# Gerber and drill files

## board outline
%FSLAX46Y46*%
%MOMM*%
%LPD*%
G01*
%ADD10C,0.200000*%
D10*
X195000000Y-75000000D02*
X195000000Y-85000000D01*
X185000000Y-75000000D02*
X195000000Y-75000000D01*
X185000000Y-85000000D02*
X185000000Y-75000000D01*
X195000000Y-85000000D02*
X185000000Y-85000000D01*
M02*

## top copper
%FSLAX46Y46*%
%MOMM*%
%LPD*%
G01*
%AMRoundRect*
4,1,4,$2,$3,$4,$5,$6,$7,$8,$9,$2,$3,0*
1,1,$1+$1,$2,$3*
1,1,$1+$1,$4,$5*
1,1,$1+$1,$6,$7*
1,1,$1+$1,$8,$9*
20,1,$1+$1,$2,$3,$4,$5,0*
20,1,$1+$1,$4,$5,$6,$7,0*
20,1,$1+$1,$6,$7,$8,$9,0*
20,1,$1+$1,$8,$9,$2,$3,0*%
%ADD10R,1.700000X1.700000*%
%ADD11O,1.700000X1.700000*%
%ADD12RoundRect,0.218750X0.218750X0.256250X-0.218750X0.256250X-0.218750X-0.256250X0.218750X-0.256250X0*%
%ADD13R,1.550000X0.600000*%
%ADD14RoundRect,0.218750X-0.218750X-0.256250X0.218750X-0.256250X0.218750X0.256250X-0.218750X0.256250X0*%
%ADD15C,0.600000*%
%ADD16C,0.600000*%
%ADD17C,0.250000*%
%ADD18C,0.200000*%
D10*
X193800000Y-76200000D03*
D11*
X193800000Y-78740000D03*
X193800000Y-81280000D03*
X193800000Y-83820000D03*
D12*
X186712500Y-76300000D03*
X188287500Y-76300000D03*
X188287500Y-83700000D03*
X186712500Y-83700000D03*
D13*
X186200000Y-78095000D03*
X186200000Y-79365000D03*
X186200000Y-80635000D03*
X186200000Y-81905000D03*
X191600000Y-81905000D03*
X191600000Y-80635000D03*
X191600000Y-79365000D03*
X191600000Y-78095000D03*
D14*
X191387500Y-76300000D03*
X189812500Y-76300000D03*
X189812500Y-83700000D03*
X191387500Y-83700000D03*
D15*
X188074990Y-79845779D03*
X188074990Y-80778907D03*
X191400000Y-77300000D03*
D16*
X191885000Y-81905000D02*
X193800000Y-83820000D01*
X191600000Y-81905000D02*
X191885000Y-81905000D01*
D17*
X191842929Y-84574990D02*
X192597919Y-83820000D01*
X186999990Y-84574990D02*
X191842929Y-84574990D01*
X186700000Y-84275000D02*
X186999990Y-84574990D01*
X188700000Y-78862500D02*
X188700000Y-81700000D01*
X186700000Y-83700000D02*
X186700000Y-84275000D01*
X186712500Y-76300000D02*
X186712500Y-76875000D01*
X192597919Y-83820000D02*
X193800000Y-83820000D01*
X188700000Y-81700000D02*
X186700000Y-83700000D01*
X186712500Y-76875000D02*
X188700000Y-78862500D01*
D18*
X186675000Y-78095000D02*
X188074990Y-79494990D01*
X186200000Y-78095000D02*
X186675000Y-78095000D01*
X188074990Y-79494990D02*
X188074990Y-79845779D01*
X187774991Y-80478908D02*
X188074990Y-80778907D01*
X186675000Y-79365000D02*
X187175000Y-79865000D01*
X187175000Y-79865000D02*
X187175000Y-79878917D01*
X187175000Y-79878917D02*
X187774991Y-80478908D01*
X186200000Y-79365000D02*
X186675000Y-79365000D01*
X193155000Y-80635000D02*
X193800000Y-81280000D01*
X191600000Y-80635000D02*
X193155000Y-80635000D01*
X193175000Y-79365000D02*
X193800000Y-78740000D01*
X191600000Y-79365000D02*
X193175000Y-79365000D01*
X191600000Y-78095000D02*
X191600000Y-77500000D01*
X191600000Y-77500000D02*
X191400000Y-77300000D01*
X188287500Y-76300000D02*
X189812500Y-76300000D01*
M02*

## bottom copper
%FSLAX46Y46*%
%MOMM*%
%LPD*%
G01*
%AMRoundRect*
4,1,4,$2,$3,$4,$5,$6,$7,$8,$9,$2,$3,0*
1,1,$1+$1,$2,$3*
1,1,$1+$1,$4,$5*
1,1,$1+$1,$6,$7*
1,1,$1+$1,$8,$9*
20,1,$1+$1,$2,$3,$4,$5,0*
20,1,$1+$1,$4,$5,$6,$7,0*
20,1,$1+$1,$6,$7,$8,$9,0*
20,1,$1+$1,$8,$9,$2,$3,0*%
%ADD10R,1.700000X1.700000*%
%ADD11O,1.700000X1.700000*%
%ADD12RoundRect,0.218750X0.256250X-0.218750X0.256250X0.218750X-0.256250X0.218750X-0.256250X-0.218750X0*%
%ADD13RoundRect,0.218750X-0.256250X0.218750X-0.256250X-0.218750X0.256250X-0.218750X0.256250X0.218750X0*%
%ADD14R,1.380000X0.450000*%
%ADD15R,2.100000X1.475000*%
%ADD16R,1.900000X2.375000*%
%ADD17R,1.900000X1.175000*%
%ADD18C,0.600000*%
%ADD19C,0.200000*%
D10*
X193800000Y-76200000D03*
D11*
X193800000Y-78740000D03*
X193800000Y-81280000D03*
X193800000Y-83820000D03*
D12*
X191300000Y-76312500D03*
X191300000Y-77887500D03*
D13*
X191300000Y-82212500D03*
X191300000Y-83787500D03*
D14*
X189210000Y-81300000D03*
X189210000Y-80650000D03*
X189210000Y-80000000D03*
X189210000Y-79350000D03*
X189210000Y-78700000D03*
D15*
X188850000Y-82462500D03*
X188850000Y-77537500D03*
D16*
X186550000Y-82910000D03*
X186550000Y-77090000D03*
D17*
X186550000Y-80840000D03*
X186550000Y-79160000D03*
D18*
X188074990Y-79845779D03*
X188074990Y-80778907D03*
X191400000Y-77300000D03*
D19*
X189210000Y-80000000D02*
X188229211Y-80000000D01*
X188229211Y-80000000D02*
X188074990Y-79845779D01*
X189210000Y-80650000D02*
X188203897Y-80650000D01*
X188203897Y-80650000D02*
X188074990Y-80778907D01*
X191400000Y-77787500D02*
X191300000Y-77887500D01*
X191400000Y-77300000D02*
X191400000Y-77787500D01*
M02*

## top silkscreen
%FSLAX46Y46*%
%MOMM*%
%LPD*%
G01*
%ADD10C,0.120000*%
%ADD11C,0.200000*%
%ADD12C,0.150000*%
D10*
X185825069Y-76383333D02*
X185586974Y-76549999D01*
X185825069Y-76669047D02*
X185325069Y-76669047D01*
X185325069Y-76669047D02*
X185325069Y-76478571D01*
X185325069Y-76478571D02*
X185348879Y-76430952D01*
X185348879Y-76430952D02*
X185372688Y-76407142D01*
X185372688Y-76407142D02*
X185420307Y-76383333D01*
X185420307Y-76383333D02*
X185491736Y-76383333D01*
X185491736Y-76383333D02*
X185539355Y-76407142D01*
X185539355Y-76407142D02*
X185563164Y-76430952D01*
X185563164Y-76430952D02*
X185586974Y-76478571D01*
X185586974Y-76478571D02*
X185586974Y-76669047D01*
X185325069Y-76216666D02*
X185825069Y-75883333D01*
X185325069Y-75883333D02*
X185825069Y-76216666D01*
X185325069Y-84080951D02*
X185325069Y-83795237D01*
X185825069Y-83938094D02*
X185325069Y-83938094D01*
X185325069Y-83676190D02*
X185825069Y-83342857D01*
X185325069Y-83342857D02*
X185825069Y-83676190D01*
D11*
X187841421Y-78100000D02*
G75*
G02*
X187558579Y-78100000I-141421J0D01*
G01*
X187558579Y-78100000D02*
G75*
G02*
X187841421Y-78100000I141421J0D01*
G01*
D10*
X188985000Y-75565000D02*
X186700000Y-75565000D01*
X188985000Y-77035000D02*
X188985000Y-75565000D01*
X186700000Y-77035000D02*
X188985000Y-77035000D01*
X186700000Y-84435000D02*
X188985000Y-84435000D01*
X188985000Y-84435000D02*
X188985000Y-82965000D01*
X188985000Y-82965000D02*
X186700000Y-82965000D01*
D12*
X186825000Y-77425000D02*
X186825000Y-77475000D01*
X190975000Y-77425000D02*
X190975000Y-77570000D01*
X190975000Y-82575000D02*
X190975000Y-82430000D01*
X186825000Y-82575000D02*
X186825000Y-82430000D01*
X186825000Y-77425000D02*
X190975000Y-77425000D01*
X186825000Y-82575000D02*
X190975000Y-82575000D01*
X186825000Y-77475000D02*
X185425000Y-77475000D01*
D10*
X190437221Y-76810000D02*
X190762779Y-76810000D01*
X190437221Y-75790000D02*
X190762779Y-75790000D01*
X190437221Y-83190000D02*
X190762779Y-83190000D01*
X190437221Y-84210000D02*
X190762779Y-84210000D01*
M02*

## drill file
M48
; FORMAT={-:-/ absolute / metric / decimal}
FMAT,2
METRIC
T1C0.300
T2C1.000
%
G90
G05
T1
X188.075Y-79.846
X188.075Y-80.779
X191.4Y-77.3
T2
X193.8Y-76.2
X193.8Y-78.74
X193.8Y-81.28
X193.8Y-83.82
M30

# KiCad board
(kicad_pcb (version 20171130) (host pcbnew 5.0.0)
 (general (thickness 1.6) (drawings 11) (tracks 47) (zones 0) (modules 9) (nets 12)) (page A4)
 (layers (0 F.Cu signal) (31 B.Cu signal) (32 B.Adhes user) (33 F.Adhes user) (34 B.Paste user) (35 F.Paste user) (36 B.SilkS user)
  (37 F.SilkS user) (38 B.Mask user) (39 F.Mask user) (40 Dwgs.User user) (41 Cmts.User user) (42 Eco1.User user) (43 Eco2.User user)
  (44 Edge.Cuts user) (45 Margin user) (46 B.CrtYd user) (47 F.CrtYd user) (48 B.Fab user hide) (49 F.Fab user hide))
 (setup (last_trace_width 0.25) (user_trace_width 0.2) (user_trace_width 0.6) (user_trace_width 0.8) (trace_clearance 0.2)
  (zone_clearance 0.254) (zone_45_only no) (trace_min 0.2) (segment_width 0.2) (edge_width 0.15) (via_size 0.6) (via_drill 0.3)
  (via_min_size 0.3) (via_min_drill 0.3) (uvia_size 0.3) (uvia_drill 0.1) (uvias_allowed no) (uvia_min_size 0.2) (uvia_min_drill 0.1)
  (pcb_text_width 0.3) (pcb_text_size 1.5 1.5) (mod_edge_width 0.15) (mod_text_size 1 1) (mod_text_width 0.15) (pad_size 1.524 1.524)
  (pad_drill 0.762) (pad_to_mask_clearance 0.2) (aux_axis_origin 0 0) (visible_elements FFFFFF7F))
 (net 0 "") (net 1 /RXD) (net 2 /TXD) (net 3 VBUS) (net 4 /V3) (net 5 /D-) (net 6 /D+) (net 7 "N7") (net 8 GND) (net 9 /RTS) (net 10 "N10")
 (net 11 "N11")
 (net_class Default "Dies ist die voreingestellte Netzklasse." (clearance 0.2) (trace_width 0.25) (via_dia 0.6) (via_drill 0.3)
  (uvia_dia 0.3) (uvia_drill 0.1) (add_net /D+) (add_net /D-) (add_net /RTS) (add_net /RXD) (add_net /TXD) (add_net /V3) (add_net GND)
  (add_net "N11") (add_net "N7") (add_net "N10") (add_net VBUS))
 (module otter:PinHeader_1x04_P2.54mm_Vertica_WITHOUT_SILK (layer F.Cu) (at 193.8 76.2)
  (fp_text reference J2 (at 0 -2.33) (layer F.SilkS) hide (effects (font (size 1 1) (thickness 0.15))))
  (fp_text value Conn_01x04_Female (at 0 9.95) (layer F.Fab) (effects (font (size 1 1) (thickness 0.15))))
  (pad 1 thru_hole rect (at 0 0) (size 1.7 1.7) (drill 1) (layers *.Cu *.Mask))
  (pad 2 thru_hole oval (at 0 2.54) (size 1.7 1.7) (drill 1) (layers *.Cu *.Mask) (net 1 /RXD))
  (pad 3 thru_hole oval (at 0 5.08) (size 1.7 1.7) (drill 1) (layers *.Cu *.Mask) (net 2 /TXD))
  (pad 4 thru_hole oval (at 0 7.62) (size 1.7 1.7) (drill 1) (layers *.Cu *.Mask) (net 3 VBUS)))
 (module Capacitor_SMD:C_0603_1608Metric (layer B.Cu) (at 191.3 77.1 90)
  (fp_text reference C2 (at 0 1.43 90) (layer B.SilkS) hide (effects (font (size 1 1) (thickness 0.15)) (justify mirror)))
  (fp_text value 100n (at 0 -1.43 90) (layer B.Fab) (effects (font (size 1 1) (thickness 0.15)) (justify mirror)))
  (pad 2 smd roundrect (at 0.7875 0 90) (size 0.875 0.95) (layers B.Cu B.Paste B.Mask) (roundrect_rratio 0.25))
  (pad 1 smd roundrect (at -0.7875 0 90) (size 0.875 0.95) (layers B.Cu B.Paste B.Mask) (roundrect_rratio 0.25) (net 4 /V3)))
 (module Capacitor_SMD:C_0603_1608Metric (layer B.Cu) (at 191.3 83 270)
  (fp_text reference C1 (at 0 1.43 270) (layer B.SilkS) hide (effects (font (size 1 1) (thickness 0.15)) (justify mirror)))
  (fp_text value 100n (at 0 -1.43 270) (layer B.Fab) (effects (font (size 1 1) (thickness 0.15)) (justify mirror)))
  (pad 1 smd roundrect (at -0.7875 0 270) (size 0.875 0.95) (layers B.Cu B.Paste B.Mask) (roundrect_rratio 0.25))
  (pad 2 smd roundrect (at 0.7875 0 270) (size 0.875 0.95) (layers B.Cu B.Paste B.Mask) (roundrect_rratio 0.25)))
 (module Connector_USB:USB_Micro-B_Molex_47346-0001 (layer B.Cu) (at 187.75 80 90)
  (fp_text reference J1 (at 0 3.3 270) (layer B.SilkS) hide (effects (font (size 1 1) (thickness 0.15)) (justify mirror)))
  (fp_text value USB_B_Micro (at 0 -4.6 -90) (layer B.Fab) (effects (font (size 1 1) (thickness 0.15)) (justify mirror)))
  (pad 1 smd rect (at -1.3 1.46 90) (size 0.45 1.38) (layers B.Cu B.Paste B.Mask))
  (pad 2 smd rect (at -0.65 1.46 90) (size 0.45 1.38) (layers B.Cu B.Paste B.Mask) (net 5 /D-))
  (pad 3 smd rect (at 0 1.46 90) (size 0.45 1.38) (layers B.Cu B.Paste B.Mask) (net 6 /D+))
  (pad 4 smd rect (at 0.65 1.46 90) (size 0.45 1.38) (layers B.Cu B.Paste B.Mask))
  (pad 5 smd rect (at 1.3 1.46 90) (size 0.45 1.38) (layers B.Cu B.Paste B.Mask))
  (pad 6 smd rect (at -2.4625 1.1 90) (size 1.475 2.1) (layers B.Cu B.Paste B.Mask))
  (pad 6 smd rect (at 2.4625 1.1 90) (size 1.475 2.1) (layers B.Cu B.Paste B.Mask))
  (pad 6 smd rect (at -2.91 -1.2 90) (size 2.375 1.9) (layers B.Cu B.Paste B.Mask))
  (pad 6 smd rect (at 2.91 -1.2 90) (size 2.375 1.9) (layers B.Cu B.Paste B.Mask))
  (pad 6 smd rect (at -0.84 -1.2 90) (size 1.175 1.9) (layers B.Cu B.Paste B.Mask))
  (pad 6 smd rect (at 0.84 -1.2 90) (size 1.175 1.9) (layers B.Cu B.Paste B.Mask)))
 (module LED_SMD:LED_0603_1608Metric (layer F.Cu) (at 187.5 76.3 180)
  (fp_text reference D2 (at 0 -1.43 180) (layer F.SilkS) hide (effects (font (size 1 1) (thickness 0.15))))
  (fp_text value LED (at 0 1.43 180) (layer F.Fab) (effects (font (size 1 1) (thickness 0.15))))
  (fp_line (start -1.485 0.735) (end 0.8 0.735) (layer F.SilkS) (width 0.12))
  (fp_line (start -1.485 -0.735) (end -1.485 0.735) (layer F.SilkS) (width 0.12))
  (fp_line (start 0.8 -0.735) (end -1.485 -0.735) (layer F.SilkS) (width 0.12))
  (pad 2 smd roundrect (at 0.7875 0 180) (size 0.875 0.95) (layers F.Cu F.Paste F.Mask) (roundrect_rratio 0.25) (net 3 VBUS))
  (pad 1 smd roundrect (at -0.7875 0 180) (size 0.875 0.95) (layers F.Cu F.Paste F.Mask) (roundrect_rratio 0.25) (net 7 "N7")))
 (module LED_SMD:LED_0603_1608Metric (layer F.Cu) (at 187.5 83.7 180)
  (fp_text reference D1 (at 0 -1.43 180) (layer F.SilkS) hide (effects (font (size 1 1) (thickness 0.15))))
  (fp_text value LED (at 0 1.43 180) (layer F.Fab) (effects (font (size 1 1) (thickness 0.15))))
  (fp_line (start 0.8 -0.735) (end -1.485 -0.735) (layer F.SilkS) (width 0.12))
  (fp_line (start -1.485 -0.735) (end -1.485 0.735) (layer F.SilkS) (width 0.12))
  (fp_line (start -1.485 0.735) (end 0.8 0.735) (layer F.SilkS) (width 0.12))
  (pad 1 smd roundrect (at -0.7875 0 180) (size 0.875 0.95) (layers F.Cu F.Paste F.Mask) (roundrect_rratio 0.25))
  (pad 2 smd roundrect (at 0.7875 0 180) (size 0.875 0.95) (layers F.Cu F.Paste F.Mask) (roundrect_rratio 0.25)))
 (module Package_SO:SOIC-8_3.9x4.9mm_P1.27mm (layer F.Cu) (at 188.9 80)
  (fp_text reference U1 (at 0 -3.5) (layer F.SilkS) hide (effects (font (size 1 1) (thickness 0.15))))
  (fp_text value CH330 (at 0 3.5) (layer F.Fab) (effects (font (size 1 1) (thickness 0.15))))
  (fp_line (start -2.075 -2.575) (end -2.075 -2.525) (layer F.SilkS) (width 0.15))
  (fp_line (start 2.075 -2.575) (end 2.075 -2.43) (layer F.SilkS) (width 0.15))
  (fp_line (start 2.075 2.575) (end 2.075 2.43) (layer F.SilkS) (width 0.15))
  (fp_line (start -2.075 2.575) (end -2.075 2.43) (layer F.SilkS) (width 0.15))
  (fp_line (start -2.075 -2.575) (end 2.075 -2.575) (layer F.SilkS) (width 0.15))
  (fp_line (start -2.075 2.575) (end 2.075 2.575) (layer F.SilkS) (width 0.15))
  (fp_line (start -2.075 -2.525) (end -3.475 -2.525) (layer F.SilkS) (width 0.15))
  (pad 1 smd rect (at -2.7 -1.905) (size 1.55 0.6) (layers F.Cu F.Paste F.Mask) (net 6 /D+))
  (pad 2 smd rect (at -2.7 -0.635) (size 1.55 0.6) (layers F.Cu F.Paste F.Mask) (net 5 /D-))
  (pad 3 smd rect (at -2.7 0.635) (size 1.55 0.6) (layers F.Cu F.Paste F.Mask))
  (pad 4 smd rect (at -2.7 1.905) (size 1.55 0.6) (layers F.Cu F.Paste F.Mask))
  (pad 5 smd rect (at 2.7 1.905) (size 1.55 0.6) (layers F.Cu F.Paste F.Mask) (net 3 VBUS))
  (pad 6 smd rect (at 2.7 0.635) (size 1.55 0.6) (layers F.Cu F.Paste F.Mask) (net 2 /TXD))
  (pad 7 smd rect (at 2.7 -0.635) (size 1.55 0.6) (layers F.Cu F.Paste F.Mask) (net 1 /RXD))
  (pad 8 smd rect (at 2.7 -1.905) (size 1.55 0.6) (layers F.Cu F.Paste F.Mask) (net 4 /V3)))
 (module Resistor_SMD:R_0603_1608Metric (layer F.Cu) (at 190.6 76.3)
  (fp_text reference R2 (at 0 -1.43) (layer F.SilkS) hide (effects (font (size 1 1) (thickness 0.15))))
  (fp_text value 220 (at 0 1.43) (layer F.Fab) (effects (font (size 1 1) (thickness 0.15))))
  (fp_line (start -0.162779 0.51) (end 0.162779 0.51) (layer F.SilkS) (width 0.12))
  (fp_line (start -0.162779 -0.51) (end 0.162779 -0.51) (layer F.SilkS) (width 0.12))
  (pad 2 smd roundrect (at 0.7875 0) (size 0.875 0.95) (layers F.Cu F.Paste F.Mask) (roundrect_rratio 0.25))
  (pad 1 smd roundrect (at -0.7875 0) (size 0.875 0.95) (layers F.Cu F.Paste F.Mask) (roundrect_rratio 0.25) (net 7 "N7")))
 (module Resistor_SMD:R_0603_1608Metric (layer F.Cu) (at 190.6 83.7)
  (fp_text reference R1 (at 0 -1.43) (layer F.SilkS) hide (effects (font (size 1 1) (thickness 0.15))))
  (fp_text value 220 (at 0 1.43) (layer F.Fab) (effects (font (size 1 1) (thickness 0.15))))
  (fp_line (start -0.162779 -0.51) (end 0.162779 -0.51) (layer F.SilkS) (width 0.12))
  (fp_line (start -0.162779 0.51) (end 0.162779 0.51) (layer F.SilkS) (width 0.12))
  (pad 1 smd roundrect (at -0.7875 0) (size 0.875 0.95) (layers F.Cu F.Paste F.Mask) (roundrect_rratio 0.25))
  (pad 2 smd roundrect (at 0.7875 0) (size 0.875 0.95) (layers F.Cu F.Paste F.Mask) (roundrect_rratio 0.25)))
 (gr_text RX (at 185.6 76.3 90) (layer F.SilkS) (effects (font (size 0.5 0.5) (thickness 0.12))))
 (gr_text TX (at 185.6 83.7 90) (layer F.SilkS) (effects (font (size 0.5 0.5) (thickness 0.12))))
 (gr_circle (center 187.7 78.1) (end 187.8 78.2) (layer F.SilkS) (width 0.2))
 (gr_line (start 195 75) (end 195 85) (layer Edge.Cuts) (width 0.2))
 (gr_line (start 185 75) (end 195 75) (layer Edge.Cuts) (width 0.2))
 (gr_line (start 185 85) (end 185 75) (layer Edge.Cuts) (width 0.2))
 (gr_line (start 195 85) (end 185 85) (layer Edge.Cuts) (width 0.2))
 (segment (start 191.885 81.905) (end 193.8 83.82) (width 0.6) (layer F.Cu) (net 3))
 (segment (start 191.6 81.905) (end 191.885 81.905) (width 0.6) (layer F.Cu) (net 3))
 (segment (start 191.842929 84.57499) (end 192.597919 83.82) (width 0.25) (layer F.Cu) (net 3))
 (segment (start 186.99999 84.57499) (end 191.842929 84.57499) (width 0.25) (layer F.Cu) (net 3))
 (segment (start 186.7 84.275) (end 186.99999 84.57499) (width 0.25) (layer F.Cu) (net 3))
 (segment (start 188.7 78.8625) (end 188.7 81.7) (width 0.25) (layer F.Cu) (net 3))
 (segment (start 186.7 83.7) (end 186.7 84.275) (width 0.25) (layer F.Cu) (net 3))
 (segment (start 186.7125 76.3) (end 186.7125 76.875) (width 0.25) (layer F.Cu) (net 3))
 (segment (start 192.597919 83.82) (end 193.8 83.82) (width 0.25) (layer F.Cu) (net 3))
 (segment (start 188.7 81.7) (end 186.7 83.7) (width 0.25) (layer F.Cu) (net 3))
 (segment (start 186.7125 76.875) (end 188.7 78.8625) (width 0.25) (layer F.Cu) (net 3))
 (segment (start 186.675 78.095) (end 188.07499 79.49499) (width 0.2) (layer F.Cu) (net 6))
 (segment (start 189.21 80) (end 188.229211 80) (width 0.2) (layer B.Cu) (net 6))
 (segment (start 188.229211 80) (end 188.07499 79.845779) (width 0.2) (layer B.Cu) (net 6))
 (segment (start 186.2 78.095) (end 186.675 78.095) (width 0.2) (layer F.Cu) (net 6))
 (segment (start 188.07499 79.49499) (end 188.07499 79.845779) (width 0.2) (layer F.Cu) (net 6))
 (segment (start 187.774991 80.478908) (end 188.07499 80.778907) (width 0.2) (layer F.Cu) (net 5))
 (segment (start 189.21 80.65) (end 188.203897 80.65) (width 0.2) (layer B.Cu) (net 5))
 (segment (start 186.675 79.365) (end 187.175 79.865) (width 0.2) (layer F.Cu) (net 5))
 (segment (start 187.175 79.865) (end 187.175 79.878917) (width 0.2) (layer F.Cu) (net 5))
 (segment (start 187.175 79.878917) (end 187.774991 80.478908) (width 0.2) (layer F.Cu) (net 5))
 (segment (start 186.2 79.365) (end 186.675 79.365) (width 0.2) (layer F.Cu) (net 5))
 (segment (start 188.203897 80.65) (end 188.07499 80.778907) (width 0.2) (layer B.Cu) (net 5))
 (segment (start 193.155 80.635) (end 193.8 81.28) (width 0.2) (layer F.Cu) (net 2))
 (segment (start 191.6 80.635) (end 193.155 80.635) (width 0.2) (layer F.Cu) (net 2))
 (segment (start 193.175 79.365) (end 193.8 78.74) (width 0.2) (layer F.Cu) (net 1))
 (segment (start 191.6 79.365) (end 193.175 79.365) (width 0.2) (layer F.Cu) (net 1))
 (segment (start 191.6 78.095) (end 191.6 77.5) (width 0.2) (layer F.Cu) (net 4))
 (segment (start 191.6 77.5) (end 191.4 77.3) (width 0.2) (layer F.Cu) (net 4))
 (segment (start 191.4 77.7875) (end 191.3 77.8875) (width 0.2) (layer B.Cu) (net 4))
 (segment (start 191.4 77.3) (end 191.4 77.7875) (width 0.2) (layer B.Cu) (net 4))
 (segment (start 188.2875 76.3) (end 189.8125 76.3) (width 0.2) (layer F.Cu) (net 7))
 (via (at 188.07499 79.845779) (size 0.6) (layers F.Cu B.Cu) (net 6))
 (via (at 188.07499 80.778907) (size 0.6) (layers F.Cu B.Cu) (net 5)) (via (at 191.4 77.3) (size 0.6) (layers F.Cu B.Cu) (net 4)))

